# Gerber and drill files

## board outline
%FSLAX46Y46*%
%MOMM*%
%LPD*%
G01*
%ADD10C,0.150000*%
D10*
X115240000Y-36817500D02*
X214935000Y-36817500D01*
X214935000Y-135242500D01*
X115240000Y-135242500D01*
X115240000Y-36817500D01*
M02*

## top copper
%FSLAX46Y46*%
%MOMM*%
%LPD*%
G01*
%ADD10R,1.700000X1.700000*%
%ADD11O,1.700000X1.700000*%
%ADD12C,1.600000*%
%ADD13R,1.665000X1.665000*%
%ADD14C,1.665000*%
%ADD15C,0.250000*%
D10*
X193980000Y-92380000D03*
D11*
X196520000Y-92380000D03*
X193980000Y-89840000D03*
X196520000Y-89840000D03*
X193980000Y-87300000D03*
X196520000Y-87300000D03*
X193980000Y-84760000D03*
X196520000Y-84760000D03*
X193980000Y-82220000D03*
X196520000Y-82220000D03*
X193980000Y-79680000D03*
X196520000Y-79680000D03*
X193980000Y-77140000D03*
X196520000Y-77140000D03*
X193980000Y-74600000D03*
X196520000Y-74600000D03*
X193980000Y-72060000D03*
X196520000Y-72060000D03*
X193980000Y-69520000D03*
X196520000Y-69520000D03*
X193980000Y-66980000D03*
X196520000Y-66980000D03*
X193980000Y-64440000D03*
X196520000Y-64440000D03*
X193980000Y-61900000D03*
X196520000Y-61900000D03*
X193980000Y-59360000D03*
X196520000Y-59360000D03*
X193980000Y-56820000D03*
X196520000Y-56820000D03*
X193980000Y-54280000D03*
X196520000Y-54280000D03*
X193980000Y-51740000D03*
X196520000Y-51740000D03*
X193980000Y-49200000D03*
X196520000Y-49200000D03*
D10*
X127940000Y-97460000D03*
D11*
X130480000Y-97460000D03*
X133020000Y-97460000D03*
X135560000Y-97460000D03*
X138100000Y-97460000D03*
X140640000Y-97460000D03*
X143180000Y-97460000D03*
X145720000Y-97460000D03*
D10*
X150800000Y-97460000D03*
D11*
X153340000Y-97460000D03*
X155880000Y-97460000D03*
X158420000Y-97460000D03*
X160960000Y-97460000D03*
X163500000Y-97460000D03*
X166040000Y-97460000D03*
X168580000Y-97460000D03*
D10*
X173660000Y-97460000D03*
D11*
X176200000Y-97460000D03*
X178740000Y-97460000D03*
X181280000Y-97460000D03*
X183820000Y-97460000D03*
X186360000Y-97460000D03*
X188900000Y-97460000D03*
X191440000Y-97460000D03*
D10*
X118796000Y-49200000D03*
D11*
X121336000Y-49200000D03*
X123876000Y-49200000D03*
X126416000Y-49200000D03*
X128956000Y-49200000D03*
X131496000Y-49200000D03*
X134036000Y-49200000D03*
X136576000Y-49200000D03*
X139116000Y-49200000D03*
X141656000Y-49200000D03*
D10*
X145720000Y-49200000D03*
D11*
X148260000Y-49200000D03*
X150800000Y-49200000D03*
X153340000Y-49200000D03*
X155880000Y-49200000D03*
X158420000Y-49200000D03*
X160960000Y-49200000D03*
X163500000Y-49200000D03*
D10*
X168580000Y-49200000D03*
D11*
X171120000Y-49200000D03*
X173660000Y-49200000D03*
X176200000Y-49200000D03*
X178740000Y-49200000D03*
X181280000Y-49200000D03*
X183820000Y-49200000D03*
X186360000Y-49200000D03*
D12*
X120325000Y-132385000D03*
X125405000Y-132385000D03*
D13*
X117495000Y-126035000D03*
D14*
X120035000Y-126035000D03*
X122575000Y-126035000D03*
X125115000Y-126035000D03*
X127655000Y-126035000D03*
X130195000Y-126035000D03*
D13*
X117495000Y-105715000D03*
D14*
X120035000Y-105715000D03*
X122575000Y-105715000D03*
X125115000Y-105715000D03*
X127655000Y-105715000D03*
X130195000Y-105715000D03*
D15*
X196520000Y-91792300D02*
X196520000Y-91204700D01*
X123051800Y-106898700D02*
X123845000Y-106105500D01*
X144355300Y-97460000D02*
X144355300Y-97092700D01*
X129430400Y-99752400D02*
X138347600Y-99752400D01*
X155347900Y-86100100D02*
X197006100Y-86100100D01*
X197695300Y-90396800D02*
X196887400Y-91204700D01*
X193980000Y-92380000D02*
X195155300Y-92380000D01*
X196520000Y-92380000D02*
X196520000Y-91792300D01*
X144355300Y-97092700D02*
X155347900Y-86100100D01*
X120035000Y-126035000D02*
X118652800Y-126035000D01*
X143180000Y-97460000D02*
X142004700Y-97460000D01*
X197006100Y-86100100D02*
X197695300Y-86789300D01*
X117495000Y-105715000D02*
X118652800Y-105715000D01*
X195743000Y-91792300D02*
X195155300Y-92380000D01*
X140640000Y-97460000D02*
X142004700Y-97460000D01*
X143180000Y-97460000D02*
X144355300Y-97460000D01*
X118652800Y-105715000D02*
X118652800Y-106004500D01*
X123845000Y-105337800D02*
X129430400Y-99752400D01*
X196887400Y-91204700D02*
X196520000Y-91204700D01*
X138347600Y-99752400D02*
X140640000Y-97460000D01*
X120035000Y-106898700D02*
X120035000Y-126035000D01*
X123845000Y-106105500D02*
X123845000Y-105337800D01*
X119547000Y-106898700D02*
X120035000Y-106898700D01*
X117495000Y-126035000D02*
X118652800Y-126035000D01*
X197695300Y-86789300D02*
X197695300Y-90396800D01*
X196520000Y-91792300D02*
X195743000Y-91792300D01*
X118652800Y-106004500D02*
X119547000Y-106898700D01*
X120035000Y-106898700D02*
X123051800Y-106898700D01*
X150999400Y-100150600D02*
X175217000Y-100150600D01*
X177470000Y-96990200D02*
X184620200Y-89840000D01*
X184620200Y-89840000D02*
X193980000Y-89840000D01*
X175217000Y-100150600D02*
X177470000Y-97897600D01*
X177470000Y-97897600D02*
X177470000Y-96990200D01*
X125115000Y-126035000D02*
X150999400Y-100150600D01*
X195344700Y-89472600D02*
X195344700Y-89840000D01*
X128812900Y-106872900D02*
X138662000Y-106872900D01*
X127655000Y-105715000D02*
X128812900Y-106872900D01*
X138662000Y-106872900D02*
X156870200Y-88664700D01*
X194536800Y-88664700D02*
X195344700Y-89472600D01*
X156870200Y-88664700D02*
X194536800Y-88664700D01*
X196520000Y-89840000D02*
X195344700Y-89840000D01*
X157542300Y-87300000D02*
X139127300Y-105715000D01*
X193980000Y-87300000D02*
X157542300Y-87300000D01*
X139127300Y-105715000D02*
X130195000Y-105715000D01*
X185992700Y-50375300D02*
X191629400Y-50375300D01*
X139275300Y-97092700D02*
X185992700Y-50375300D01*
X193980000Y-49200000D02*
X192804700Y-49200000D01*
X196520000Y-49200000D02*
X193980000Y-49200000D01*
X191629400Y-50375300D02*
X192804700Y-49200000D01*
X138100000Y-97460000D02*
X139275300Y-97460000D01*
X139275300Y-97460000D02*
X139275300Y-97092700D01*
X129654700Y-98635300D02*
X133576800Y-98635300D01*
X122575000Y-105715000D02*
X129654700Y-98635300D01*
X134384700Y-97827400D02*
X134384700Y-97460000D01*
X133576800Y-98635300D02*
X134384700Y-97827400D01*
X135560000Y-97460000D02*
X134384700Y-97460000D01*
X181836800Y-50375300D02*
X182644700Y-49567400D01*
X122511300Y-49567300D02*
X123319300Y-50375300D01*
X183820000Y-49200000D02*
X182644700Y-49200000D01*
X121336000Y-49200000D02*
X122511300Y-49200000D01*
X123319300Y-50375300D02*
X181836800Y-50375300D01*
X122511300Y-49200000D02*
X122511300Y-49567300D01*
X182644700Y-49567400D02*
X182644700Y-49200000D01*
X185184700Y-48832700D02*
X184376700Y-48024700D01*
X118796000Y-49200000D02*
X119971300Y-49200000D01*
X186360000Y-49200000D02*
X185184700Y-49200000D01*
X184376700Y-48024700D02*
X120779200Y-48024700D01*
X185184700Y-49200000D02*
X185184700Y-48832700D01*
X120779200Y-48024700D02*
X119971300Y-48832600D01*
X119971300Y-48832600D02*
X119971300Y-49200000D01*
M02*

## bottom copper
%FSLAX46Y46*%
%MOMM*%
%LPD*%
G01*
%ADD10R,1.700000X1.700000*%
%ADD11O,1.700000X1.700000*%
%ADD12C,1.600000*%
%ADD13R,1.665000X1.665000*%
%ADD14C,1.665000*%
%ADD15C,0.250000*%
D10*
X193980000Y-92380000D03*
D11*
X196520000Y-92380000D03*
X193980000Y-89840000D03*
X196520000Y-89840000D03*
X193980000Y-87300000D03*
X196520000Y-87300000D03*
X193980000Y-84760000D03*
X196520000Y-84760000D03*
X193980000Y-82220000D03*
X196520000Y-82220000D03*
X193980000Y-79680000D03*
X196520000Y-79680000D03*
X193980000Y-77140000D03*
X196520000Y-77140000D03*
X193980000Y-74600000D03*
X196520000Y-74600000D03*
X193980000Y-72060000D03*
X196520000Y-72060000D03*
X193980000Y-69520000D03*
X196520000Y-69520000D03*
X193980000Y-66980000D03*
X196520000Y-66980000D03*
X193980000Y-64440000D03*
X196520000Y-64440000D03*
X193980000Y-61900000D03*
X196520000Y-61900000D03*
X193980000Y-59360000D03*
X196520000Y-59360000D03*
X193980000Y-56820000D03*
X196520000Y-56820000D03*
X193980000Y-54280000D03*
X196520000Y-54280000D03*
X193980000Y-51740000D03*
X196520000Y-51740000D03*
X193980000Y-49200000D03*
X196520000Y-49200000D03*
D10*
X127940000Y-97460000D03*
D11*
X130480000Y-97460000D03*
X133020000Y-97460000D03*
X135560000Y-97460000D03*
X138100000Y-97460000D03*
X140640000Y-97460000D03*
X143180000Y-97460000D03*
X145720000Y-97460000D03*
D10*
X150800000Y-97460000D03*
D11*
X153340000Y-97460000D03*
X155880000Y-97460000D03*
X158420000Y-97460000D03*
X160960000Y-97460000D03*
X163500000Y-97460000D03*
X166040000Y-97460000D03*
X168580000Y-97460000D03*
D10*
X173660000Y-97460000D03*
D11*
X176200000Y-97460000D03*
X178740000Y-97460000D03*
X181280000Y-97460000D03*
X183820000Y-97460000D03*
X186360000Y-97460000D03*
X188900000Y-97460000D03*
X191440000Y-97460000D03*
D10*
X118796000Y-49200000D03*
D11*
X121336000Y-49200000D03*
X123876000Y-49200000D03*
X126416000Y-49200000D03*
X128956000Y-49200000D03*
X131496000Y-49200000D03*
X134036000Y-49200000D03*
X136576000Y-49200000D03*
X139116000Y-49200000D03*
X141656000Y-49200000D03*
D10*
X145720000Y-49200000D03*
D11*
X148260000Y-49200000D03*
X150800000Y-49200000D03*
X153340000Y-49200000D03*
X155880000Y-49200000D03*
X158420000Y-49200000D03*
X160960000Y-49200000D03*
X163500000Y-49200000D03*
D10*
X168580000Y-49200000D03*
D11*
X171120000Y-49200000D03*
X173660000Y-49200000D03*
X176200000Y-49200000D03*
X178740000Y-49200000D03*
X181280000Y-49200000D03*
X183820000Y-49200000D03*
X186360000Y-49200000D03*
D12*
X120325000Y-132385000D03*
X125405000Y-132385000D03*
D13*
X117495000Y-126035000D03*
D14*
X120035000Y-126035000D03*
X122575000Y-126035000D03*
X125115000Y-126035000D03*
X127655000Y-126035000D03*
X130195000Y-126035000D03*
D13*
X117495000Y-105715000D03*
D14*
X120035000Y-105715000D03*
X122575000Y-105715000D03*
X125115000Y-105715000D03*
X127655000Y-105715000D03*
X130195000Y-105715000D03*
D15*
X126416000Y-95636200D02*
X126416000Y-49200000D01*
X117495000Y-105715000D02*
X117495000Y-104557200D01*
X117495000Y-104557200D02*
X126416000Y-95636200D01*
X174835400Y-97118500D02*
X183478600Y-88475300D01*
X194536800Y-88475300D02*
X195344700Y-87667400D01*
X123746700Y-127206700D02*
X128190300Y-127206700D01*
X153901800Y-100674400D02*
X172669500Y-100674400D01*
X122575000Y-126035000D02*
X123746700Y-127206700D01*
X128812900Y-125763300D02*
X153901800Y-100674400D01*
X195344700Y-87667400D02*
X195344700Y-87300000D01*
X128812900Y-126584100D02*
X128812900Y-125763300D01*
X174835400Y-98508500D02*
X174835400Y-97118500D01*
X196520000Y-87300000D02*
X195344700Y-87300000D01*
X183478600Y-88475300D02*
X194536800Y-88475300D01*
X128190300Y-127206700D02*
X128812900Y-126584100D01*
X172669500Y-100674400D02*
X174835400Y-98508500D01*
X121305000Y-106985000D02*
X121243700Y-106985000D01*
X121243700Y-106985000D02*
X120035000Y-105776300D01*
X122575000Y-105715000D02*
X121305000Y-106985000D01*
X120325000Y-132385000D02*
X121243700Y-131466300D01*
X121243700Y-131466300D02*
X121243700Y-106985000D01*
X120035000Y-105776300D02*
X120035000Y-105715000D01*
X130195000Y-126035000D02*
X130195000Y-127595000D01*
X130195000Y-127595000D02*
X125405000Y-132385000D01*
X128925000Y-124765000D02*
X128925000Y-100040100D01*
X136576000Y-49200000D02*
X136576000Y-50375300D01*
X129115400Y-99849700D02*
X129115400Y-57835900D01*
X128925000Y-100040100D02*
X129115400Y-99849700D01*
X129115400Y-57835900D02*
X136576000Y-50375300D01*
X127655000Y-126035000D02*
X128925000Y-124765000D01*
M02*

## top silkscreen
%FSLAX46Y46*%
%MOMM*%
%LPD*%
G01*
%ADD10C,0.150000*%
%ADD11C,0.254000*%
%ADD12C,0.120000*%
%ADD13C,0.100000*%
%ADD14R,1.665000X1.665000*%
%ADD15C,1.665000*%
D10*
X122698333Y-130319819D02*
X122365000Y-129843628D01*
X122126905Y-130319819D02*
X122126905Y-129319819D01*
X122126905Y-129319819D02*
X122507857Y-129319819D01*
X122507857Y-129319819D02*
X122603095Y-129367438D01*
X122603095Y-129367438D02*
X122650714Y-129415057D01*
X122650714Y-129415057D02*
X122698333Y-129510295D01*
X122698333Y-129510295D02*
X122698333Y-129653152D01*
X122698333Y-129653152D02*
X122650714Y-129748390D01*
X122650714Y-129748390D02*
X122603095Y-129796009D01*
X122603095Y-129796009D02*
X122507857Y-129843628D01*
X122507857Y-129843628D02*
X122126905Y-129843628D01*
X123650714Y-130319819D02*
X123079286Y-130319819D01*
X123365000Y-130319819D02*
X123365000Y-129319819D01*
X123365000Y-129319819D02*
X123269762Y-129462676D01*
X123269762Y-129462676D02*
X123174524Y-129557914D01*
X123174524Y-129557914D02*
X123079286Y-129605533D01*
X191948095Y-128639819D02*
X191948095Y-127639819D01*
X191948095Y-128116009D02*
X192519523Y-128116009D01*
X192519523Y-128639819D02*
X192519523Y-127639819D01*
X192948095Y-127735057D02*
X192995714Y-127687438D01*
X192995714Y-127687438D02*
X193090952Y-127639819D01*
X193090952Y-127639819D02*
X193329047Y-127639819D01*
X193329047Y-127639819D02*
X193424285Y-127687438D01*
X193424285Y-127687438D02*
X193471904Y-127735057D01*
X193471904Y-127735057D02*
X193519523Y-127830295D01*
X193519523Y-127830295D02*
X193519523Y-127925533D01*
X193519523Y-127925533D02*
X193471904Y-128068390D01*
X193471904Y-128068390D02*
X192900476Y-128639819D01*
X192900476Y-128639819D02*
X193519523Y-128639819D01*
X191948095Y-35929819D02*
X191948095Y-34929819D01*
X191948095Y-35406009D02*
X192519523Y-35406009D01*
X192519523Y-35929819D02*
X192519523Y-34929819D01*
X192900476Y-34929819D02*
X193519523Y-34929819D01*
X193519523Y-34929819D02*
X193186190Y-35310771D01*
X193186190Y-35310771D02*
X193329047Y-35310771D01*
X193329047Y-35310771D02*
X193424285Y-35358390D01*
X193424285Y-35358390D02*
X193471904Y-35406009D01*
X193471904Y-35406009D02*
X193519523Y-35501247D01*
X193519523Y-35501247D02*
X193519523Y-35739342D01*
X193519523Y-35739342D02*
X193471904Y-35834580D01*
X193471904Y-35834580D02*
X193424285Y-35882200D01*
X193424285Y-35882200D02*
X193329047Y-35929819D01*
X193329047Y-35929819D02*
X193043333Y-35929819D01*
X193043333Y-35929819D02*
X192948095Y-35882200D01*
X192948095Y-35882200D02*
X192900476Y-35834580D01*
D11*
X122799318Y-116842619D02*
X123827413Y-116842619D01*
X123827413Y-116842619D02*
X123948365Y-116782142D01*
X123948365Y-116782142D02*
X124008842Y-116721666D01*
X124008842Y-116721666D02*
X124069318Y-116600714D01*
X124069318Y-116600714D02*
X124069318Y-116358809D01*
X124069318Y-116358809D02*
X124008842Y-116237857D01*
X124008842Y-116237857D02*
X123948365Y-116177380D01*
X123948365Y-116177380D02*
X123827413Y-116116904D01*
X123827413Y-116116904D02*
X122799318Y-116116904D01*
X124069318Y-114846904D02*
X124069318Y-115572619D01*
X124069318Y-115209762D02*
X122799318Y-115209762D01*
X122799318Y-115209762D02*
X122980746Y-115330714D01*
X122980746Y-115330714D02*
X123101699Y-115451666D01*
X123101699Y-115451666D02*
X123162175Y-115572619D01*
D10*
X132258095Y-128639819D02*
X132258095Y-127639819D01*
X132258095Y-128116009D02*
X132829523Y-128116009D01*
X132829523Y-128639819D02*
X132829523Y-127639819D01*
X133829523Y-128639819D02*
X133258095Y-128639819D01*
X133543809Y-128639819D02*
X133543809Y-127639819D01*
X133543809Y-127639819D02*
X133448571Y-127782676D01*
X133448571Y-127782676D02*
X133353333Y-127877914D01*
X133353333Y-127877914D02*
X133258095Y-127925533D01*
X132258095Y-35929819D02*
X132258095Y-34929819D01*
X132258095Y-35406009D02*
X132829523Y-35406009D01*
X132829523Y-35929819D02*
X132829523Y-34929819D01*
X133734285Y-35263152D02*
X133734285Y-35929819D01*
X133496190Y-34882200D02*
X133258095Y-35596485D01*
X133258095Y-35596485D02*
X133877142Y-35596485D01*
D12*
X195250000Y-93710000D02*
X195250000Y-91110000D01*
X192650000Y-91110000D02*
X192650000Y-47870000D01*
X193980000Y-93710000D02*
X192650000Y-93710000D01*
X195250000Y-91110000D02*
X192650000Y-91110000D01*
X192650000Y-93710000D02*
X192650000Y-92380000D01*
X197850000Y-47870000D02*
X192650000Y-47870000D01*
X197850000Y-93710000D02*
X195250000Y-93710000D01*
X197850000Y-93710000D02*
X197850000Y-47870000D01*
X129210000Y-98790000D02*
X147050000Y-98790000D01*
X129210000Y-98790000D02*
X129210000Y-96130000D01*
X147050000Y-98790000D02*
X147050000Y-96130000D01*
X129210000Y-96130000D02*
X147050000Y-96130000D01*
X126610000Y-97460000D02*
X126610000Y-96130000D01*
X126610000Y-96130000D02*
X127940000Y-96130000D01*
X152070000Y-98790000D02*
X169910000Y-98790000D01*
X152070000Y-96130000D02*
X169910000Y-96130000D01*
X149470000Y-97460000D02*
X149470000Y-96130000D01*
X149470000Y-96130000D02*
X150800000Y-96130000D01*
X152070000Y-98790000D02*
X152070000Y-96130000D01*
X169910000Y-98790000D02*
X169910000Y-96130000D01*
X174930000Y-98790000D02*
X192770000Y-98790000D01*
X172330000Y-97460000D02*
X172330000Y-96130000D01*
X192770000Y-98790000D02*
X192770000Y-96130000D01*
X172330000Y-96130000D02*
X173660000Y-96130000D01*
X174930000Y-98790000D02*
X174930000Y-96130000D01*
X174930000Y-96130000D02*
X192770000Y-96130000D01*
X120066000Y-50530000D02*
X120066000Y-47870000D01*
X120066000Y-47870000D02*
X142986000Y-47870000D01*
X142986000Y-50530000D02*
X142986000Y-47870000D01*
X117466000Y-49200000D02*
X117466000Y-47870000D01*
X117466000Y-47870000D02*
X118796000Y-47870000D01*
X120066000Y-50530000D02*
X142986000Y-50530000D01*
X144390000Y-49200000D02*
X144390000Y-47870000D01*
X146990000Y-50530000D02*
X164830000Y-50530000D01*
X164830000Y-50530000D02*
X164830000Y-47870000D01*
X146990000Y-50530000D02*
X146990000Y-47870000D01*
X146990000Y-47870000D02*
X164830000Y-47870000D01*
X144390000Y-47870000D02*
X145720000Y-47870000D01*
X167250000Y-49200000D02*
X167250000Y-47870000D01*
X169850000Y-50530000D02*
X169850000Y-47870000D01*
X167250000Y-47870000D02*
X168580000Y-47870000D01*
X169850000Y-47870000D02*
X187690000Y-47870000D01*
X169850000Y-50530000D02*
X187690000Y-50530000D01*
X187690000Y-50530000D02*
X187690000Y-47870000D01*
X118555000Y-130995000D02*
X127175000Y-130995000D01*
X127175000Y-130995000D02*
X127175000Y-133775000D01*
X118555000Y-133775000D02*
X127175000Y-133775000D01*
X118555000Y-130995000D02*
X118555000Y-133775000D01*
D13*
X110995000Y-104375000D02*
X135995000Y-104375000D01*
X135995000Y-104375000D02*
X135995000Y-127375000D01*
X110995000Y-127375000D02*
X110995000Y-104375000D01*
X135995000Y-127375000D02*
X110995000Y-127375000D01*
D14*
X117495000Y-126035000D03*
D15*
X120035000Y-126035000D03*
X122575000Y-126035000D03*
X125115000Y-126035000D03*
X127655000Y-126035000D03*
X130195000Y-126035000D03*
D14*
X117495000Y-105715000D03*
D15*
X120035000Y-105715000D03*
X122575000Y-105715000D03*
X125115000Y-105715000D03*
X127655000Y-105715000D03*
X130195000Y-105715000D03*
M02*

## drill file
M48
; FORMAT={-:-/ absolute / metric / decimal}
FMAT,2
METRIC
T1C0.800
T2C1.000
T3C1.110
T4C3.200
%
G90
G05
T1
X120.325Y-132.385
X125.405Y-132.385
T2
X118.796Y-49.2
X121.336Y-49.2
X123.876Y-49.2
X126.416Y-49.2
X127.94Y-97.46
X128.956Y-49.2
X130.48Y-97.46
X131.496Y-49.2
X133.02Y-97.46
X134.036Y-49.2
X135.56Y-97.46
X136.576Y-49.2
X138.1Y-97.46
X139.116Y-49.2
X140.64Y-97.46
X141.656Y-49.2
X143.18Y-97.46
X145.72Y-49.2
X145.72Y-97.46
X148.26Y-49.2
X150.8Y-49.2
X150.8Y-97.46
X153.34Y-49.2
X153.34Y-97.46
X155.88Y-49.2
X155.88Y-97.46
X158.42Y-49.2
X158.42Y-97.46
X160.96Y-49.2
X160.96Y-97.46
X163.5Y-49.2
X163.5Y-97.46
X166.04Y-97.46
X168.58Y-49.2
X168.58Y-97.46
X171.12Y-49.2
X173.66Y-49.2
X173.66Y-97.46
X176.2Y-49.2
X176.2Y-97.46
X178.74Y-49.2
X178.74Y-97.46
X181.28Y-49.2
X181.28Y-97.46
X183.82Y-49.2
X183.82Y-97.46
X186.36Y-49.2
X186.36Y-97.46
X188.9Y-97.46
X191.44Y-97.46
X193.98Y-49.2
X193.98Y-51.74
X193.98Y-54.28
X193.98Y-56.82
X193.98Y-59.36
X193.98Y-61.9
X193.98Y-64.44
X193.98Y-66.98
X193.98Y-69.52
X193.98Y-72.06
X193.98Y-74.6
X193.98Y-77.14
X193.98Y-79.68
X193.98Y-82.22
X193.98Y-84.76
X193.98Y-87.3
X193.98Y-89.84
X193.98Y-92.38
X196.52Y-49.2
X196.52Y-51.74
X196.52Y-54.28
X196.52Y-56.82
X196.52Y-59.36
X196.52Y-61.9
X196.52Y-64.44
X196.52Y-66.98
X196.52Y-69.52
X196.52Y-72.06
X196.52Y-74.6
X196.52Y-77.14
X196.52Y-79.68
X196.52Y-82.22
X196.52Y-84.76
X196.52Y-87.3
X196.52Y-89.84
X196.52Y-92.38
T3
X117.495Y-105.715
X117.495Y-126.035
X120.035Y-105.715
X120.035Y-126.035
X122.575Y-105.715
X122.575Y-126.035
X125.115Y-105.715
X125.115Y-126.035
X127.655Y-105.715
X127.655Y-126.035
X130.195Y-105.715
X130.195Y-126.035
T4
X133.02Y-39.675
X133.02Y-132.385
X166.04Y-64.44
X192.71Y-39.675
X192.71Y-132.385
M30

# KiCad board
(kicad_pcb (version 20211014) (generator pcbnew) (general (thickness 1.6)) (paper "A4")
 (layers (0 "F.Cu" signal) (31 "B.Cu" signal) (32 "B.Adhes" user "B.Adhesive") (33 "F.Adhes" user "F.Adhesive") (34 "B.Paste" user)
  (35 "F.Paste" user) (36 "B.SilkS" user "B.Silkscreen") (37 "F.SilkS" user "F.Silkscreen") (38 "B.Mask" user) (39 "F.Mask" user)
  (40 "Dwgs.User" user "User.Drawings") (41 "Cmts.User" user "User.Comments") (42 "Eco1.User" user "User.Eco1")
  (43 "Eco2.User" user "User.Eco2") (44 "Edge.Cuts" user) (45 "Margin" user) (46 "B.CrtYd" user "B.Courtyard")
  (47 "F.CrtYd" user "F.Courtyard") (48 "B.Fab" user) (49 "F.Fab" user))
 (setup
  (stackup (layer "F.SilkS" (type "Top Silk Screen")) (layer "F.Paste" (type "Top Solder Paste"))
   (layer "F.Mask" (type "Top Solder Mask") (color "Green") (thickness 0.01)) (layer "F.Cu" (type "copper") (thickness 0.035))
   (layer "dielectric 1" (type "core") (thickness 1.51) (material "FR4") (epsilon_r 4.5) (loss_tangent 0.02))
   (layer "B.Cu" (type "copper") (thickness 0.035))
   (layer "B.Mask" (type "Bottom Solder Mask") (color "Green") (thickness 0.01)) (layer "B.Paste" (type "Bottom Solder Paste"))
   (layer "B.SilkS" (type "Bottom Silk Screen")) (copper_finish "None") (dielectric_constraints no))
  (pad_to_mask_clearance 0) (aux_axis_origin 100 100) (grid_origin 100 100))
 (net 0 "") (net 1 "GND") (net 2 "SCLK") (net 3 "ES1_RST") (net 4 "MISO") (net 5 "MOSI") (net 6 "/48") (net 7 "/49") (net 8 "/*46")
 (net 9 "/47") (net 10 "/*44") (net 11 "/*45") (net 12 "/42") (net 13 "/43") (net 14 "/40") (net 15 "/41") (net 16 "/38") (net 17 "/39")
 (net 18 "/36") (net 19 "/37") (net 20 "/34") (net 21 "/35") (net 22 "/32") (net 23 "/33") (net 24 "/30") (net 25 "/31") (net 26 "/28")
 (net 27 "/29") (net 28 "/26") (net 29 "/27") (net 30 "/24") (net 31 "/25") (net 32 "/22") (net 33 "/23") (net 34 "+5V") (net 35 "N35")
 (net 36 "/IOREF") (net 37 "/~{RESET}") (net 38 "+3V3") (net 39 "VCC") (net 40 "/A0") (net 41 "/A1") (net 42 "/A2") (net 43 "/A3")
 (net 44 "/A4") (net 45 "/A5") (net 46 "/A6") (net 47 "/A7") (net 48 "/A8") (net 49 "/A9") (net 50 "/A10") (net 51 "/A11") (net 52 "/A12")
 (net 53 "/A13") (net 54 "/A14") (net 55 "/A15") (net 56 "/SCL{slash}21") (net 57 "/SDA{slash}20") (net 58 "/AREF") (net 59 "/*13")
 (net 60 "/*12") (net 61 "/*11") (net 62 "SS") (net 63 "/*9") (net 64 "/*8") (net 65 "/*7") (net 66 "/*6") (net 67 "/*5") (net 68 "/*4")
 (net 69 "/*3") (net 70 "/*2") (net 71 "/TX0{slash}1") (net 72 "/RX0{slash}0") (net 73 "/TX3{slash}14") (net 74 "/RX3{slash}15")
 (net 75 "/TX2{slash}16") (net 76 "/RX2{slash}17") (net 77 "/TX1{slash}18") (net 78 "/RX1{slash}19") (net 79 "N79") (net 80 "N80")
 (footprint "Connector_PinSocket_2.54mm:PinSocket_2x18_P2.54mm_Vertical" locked (layer "F.Cu") (at 193.98 92.38 180)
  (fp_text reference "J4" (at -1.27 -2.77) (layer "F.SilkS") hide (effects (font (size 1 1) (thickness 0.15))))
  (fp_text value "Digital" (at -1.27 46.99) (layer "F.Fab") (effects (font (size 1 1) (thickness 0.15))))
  (fp_line (start -1.27 -1.33) (end -1.27 1.27) (layer "F.SilkS") (width 0.12))
  (fp_line (start 1.33 1.27) (end 1.33 44.51) (layer "F.SilkS") (width 0.12))
  (fp_line (start 0 -1.33) (end 1.33 -1.33) (layer "F.SilkS") (width 0.12))
  (fp_line (start -1.27 1.27) (end 1.33 1.27) (layer "F.SilkS") (width 0.12))
  (fp_line (start 1.33 -1.33) (end 1.33 0) (layer "F.SilkS") (width 0.12))
  (fp_line (start -3.87 44.51) (end 1.33 44.51) (layer "F.SilkS") (width 0.12))
  (fp_line (start -3.87 -1.33) (end -1.27 -1.33) (layer "F.SilkS") (width 0.12))
  (fp_line (start -3.87 -1.33) (end -3.87 44.51) (layer "F.SilkS") (width 0.12))
  (pad "1" thru_hole rect locked (at 0 0 180) (size 1.7 1.7) (drill 1) (layers *.Cu *.Mask) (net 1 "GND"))
  (pad "2" thru_hole oval locked (at -2.54 0 180) (size 1.7 1.7) (drill 1) (layers *.Cu *.Mask) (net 1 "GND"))
  (pad "3" thru_hole oval locked (at 0 2.54 180) (size 1.7 1.7) (drill 1) (layers *.Cu *.Mask) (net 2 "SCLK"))
  (pad "4" thru_hole oval locked (at -2.54 2.54 180) (size 1.7 1.7) (drill 1) (layers *.Cu *.Mask) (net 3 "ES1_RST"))
  (pad "5" thru_hole oval locked (at 0 5.08 180) (size 1.7 1.7) (drill 1) (layers *.Cu *.Mask) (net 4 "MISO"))
  (pad "6" thru_hole oval locked (at -2.54 5.08 180) (size 1.7 1.7) (drill 1) (layers *.Cu *.Mask) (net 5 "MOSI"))
  (pad "7" thru_hole oval locked (at 0 7.62 180) (size 1.7 1.7) (drill 1) (layers *.Cu *.Mask) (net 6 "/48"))
  (pad "8" thru_hole oval locked (at -2.54 7.62 180) (size 1.7 1.7) (drill 1) (layers *.Cu *.Mask) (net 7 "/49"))
  (pad "9" thru_hole oval locked (at 0 10.16 180) (size 1.7 1.7) (drill 1) (layers *.Cu *.Mask) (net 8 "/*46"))
  (pad "10" thru_hole oval locked (at -2.54 10.16 180) (size 1.7 1.7) (drill 1) (layers *.Cu *.Mask) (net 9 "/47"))
  (pad "11" thru_hole oval locked (at 0 12.7 180) (size 1.7 1.7) (drill 1) (layers *.Cu *.Mask) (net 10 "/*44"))
  (pad "12" thru_hole oval locked (at -2.54 12.7 180) (size 1.7 1.7) (drill 1) (layers *.Cu *.Mask) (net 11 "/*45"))
  (pad "13" thru_hole oval locked (at 0 15.24 180) (size 1.7 1.7) (drill 1) (layers *.Cu *.Mask) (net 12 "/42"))
  (pad "14" thru_hole oval locked (at -2.54 15.24 180) (size 1.7 1.7) (drill 1) (layers *.Cu *.Mask) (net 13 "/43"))
  (pad "15" thru_hole oval locked (at 0 17.78 180) (size 1.7 1.7) (drill 1) (layers *.Cu *.Mask) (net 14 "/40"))
  (pad "16" thru_hole oval locked (at -2.54 17.78 180) (size 1.7 1.7) (drill 1) (layers *.Cu *.Mask) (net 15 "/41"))
  (pad "17" thru_hole oval locked (at 0 20.32 180) (size 1.7 1.7) (drill 1) (layers *.Cu *.Mask) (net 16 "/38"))
  (pad "18" thru_hole oval locked (at -2.54 20.32 180) (size 1.7 1.7) (drill 1) (layers *.Cu *.Mask) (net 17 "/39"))
  (pad "19" thru_hole oval locked (at 0 22.86 180) (size 1.7 1.7) (drill 1) (layers *.Cu *.Mask) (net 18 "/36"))
  (pad "20" thru_hole oval locked (at -2.54 22.86 180) (size 1.7 1.7) (drill 1) (layers *.Cu *.Mask) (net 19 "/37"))
  (pad "21" thru_hole oval locked (at 0 25.4 180) (size 1.7 1.7) (drill 1) (layers *.Cu *.Mask) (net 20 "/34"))
  (pad "22" thru_hole oval locked (at -2.54 25.4 180) (size 1.7 1.7) (drill 1) (layers *.Cu *.Mask) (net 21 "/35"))
  (pad "23" thru_hole oval locked (at 0 27.94 180) (size 1.7 1.7) (drill 1) (layers *.Cu *.Mask) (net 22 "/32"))
  (pad "24" thru_hole oval locked (at -2.54 27.94 180) (size 1.7 1.7) (drill 1) (layers *.Cu *.Mask) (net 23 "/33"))
  (pad "25" thru_hole oval locked (at 0 30.48 180) (size 1.7 1.7) (drill 1) (layers *.Cu *.Mask) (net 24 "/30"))
  (pad "26" thru_hole oval locked (at -2.54 30.48 180) (size 1.7 1.7) (drill 1) (layers *.Cu *.Mask) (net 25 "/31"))
  (pad "27" thru_hole oval locked (at 0 33.02 180) (size 1.7 1.7) (drill 1) (layers *.Cu *.Mask) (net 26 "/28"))
  (pad "28" thru_hole oval locked (at -2.54 33.02 180) (size 1.7 1.7) (drill 1) (layers *.Cu *.Mask) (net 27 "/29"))
  (pad "29" thru_hole oval locked (at 0 35.56 180) (size 1.7 1.7) (drill 1) (layers *.Cu *.Mask) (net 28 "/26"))
  (pad "30" thru_hole oval locked (at -2.54 35.56 180) (size 1.7 1.7) (drill 1) (layers *.Cu *.Mask) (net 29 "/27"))
  (pad "31" thru_hole oval locked (at 0 38.1 180) (size 1.7 1.7) (drill 1) (layers *.Cu *.Mask) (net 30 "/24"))
  (pad "32" thru_hole oval locked (at -2.54 38.1 180) (size 1.7 1.7) (drill 1) (layers *.Cu *.Mask) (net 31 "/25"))
  (pad "33" thru_hole oval locked (at 0 40.64 180) (size 1.7 1.7) (drill 1) (layers *.Cu *.Mask) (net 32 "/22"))
  (pad "34" thru_hole oval locked (at -2.54 40.64 180) (size 1.7 1.7) (drill 1) (layers *.Cu *.Mask) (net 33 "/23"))
  (pad "35" thru_hole oval locked (at 0 43.18 180) (size 1.7 1.7) (drill 1) (layers *.Cu *.Mask) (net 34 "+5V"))
  (pad "36" thru_hole oval locked (at -2.54 43.18 180) (size 1.7 1.7) (drill 1) (layers *.Cu *.Mask) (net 34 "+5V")))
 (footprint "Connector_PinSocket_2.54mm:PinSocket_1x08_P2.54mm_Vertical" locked (layer "F.Cu") (at 127.94 97.46 90)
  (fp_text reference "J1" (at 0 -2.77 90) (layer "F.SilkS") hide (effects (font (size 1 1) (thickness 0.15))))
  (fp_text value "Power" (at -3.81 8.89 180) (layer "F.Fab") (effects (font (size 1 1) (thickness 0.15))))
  (fp_line (start -1.33 1.27) (end -1.33 19.11) (layer "F.SilkS") (width 0.12))
  (fp_line (start -1.33 1.27) (end 1.33 1.27) (layer "F.SilkS") (width 0.12))
  (fp_line (start -1.33 19.11) (end 1.33 19.11) (layer "F.SilkS") (width 0.12))
  (fp_line (start 1.33 1.27) (end 1.33 19.11) (layer "F.SilkS") (width 0.12))
  (fp_line (start 0 -1.33) (end 1.33 -1.33) (layer "F.SilkS") (width 0.12))
  (fp_line (start 1.33 -1.33) (end 1.33 0) (layer "F.SilkS") (width 0.12))
  (pad "1" thru_hole rect locked (at 0 0 90) (size 1.7 1.7) (drill 1) (layers *.Cu *.Mask) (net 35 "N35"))
  (pad "2" thru_hole oval locked (at 0 2.54 90) (size 1.7 1.7) (drill 1) (layers *.Cu *.Mask) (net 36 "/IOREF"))
  (pad "3" thru_hole oval locked (at 0 5.08 90) (size 1.7 1.7) (drill 1) (layers *.Cu *.Mask) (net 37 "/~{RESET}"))
  (pad "4" thru_hole oval locked (at 0 7.62 90) (size 1.7 1.7) (drill 1) (layers *.Cu *.Mask) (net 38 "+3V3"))
  (pad "5" thru_hole oval locked (at 0 10.16 90) (size 1.7 1.7) (drill 1) (layers *.Cu *.Mask) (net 34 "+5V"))
  (pad "6" thru_hole oval locked (at 0 12.7 90) (size 1.7 1.7) (drill 1) (layers *.Cu *.Mask) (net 1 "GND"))
  (pad "7" thru_hole oval locked (at 0 15.24 90) (size 1.7 1.7) (drill 1) (layers *.Cu *.Mask) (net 1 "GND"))
  (pad "8" thru_hole oval locked (at 0 17.78 90) (size 1.7 1.7) (drill 1) (layers *.Cu *.Mask) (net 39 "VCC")))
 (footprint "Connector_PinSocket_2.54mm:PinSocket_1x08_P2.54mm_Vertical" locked (layer "F.Cu") (at 150.8 97.46 90)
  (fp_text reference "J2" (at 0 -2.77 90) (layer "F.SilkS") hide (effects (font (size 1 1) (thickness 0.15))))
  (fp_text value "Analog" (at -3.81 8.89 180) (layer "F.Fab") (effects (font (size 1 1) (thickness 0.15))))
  (fp_line (start -1.33 1.27) (end -1.33 19.11) (layer "F.SilkS") (width 0.12))
  (fp_line (start 1.33 1.27) (end 1.33 19.11) (layer "F.SilkS") (width 0.12))
  (fp_line (start 0 -1.33) (end 1.33 -1.33) (layer "F.SilkS") (width 0.12))
  (fp_line (start 1.33 -1.33) (end 1.33 0) (layer "F.SilkS") (width 0.12))
  (fp_line (start -1.33 1.27) (end 1.33 1.27) (layer "F.SilkS") (width 0.12))
  (fp_line (start -1.33 19.11) (end 1.33 19.11) (layer "F.SilkS") (width 0.12))
  (pad "1" thru_hole rect locked (at 0 0 90) (size 1.7 1.7) (drill 1) (layers *.Cu *.Mask) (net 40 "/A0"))
  (pad "2" thru_hole oval locked (at 0 2.54 90) (size 1.7 1.7) (drill 1) (layers *.Cu *.Mask) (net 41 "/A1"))
  (pad "3" thru_hole oval locked (at 0 5.08 90) (size 1.7 1.7) (drill 1) (layers *.Cu *.Mask) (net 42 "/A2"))
  (pad "4" thru_hole oval locked (at 0 7.62 90) (size 1.7 1.7) (drill 1) (layers *.Cu *.Mask) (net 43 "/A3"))
  (pad "5" thru_hole oval locked (at 0 10.16 90) (size 1.7 1.7) (drill 1) (layers *.Cu *.Mask) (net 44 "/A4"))
  (pad "6" thru_hole oval locked (at 0 12.7 90) (size 1.7 1.7) (drill 1) (layers *.Cu *.Mask) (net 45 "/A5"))
  (pad "7" thru_hole oval locked (at 0 15.24 90) (size 1.7 1.7) (drill 1) (layers *.Cu *.Mask) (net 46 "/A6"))
  (pad "8" thru_hole oval locked (at 0 17.78 90) (size 1.7 1.7) (drill 1) (layers *.Cu *.Mask) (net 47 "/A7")))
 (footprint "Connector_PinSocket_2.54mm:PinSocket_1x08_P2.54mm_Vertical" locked (layer "F.Cu") (at 173.66 97.46 90)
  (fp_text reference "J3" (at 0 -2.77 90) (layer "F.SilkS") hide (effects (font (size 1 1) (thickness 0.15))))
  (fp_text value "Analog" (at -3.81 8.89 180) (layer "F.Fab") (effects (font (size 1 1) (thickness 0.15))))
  (fp_line (start -1.33 1.27) (end -1.33 19.11) (layer "F.SilkS") (width 0.12))
  (fp_line (start 0 -1.33) (end 1.33 -1.33) (layer "F.SilkS") (width 0.12))
  (fp_line (start -1.33 19.11) (end 1.33 19.11) (layer "F.SilkS") (width 0.12))
  (fp_line (start 1.33 -1.33) (end 1.33 0) (layer "F.SilkS") (width 0.12))
  (fp_line (start -1.33 1.27) (end 1.33 1.27) (layer "F.SilkS") (width 0.12))
  (fp_line (start 1.33 1.27) (end 1.33 19.11) (layer "F.SilkS") (width 0.12))
  (pad "1" thru_hole rect locked (at 0 0 90) (size 1.7 1.7) (drill 1) (layers *.Cu *.Mask) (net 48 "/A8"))
  (pad "2" thru_hole oval locked (at 0 2.54 90) (size 1.7 1.7) (drill 1) (layers *.Cu *.Mask) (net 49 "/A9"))
  (pad "3" thru_hole oval locked (at 0 5.08 90) (size 1.7 1.7) (drill 1) (layers *.Cu *.Mask) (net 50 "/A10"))
  (pad "4" thru_hole oval locked (at 0 7.62 90) (size 1.7 1.7) (drill 1) (layers *.Cu *.Mask) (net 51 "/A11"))
  (pad "5" thru_hole oval locked (at 0 10.16 90) (size 1.7 1.7) (drill 1) (layers *.Cu *.Mask) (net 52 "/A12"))
  (pad "6" thru_hole oval locked (at 0 12.7 90) (size 1.7 1.7) (drill 1) (layers *.Cu *.Mask) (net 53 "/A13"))
  (pad "7" thru_hole oval locked (at 0 15.24 90) (size 1.7 1.7) (drill 1) (layers *.Cu *.Mask) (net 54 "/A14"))
  (pad "8" thru_hole oval locked (at 0 17.78 90) (size 1.7 1.7) (drill 1) (layers *.Cu *.Mask) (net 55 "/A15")))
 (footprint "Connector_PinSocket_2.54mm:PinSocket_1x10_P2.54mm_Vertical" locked (layer "F.Cu") (at 118.796 49.2 90)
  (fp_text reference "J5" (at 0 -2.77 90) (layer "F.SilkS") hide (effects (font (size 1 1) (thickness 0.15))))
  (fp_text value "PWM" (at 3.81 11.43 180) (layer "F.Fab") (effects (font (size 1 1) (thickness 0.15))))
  (fp_line (start -1.33 1.27) (end 1.33 1.27) (layer "F.SilkS") (width 0.12))
  (fp_line (start 1.33 1.27) (end 1.33 24.19) (layer "F.SilkS") (width 0.12))
  (fp_line (start -1.33 24.19) (end 1.33 24.19) (layer "F.SilkS") (width 0.12))
  (fp_line (start 0 -1.33) (end 1.33 -1.33) (layer "F.SilkS") (width 0.12))
  (fp_line (start 1.33 -1.33) (end 1.33 0) (layer "F.SilkS") (width 0.12))
  (fp_line (start -1.33 1.27) (end -1.33 24.19) (layer "F.SilkS") (width 0.12))
  (pad "1" thru_hole rect locked (at 0 0 90) (size 1.7 1.7) (drill 1) (layers *.Cu *.Mask) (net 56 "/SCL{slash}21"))
  (pad "2" thru_hole oval locked (at 0 2.54 90) (size 1.7 1.7) (drill 1) (layers *.Cu *.Mask) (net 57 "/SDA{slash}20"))
  (pad "3" thru_hole oval locked (at 0 5.08 90) (size 1.7 1.7) (drill 1) (layers *.Cu *.Mask) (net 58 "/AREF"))
  (pad "4" thru_hole oval locked (at 0 7.62 90) (size 1.7 1.7) (drill 1) (layers *.Cu *.Mask) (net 1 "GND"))
  (pad "5" thru_hole oval locked (at 0 10.16 90) (size 1.7 1.7) (drill 1) (layers *.Cu *.Mask) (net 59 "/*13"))
  (pad "6" thru_hole oval locked (at 0 12.7 90) (size 1.7 1.7) (drill 1) (layers *.Cu *.Mask) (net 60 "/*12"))
  (pad "7" thru_hole oval locked (at 0 15.24 90) (size 1.7 1.7) (drill 1) (layers *.Cu *.Mask) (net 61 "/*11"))
  (pad "8" thru_hole oval locked (at 0 17.78 90) (size 1.7 1.7) (drill 1) (layers *.Cu *.Mask) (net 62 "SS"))
  (pad "9" thru_hole oval locked (at 0 20.32 90) (size 1.7 1.7) (drill 1) (layers *.Cu *.Mask) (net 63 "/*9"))
  (pad "10" thru_hole oval locked (at 0 22.86 90) (size 1.7 1.7) (drill 1) (layers *.Cu *.Mask) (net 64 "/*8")))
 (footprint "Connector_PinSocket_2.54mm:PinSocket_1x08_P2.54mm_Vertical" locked (layer "F.Cu") (at 145.72 49.2 90)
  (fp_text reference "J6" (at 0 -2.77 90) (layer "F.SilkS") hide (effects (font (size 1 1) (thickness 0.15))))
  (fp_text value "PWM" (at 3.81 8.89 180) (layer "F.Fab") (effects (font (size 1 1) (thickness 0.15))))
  (fp_line (start 0 -1.33) (end 1.33 -1.33) (layer "F.SilkS") (width 0.12))
  (fp_line (start -1.33 1.27) (end -1.33 19.11) (layer "F.SilkS") (width 0.12))
  (fp_line (start -1.33 19.11) (end 1.33 19.11) (layer "F.SilkS") (width 0.12))
  (fp_line (start -1.33 1.27) (end 1.33 1.27) (layer "F.SilkS") (width 0.12))
  (fp_line (start 1.33 1.27) (end 1.33 19.11) (layer "F.SilkS") (width 0.12))
  (fp_line (start 1.33 -1.33) (end 1.33 0) (layer "F.SilkS") (width 0.12))
  (pad "1" thru_hole rect locked (at 0 0 90) (size 1.7 1.7) (drill 1) (layers *.Cu *.Mask) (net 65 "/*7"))
  (pad "2" thru_hole oval locked (at 0 2.54 90) (size 1.7 1.7) (drill 1) (layers *.Cu *.Mask) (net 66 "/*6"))
  (pad "3" thru_hole oval locked (at 0 5.08 90) (size 1.7 1.7) (drill 1) (layers *.Cu *.Mask) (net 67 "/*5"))
  (pad "4" thru_hole oval locked (at 0 7.62 90) (size 1.7 1.7) (drill 1) (layers *.Cu *.Mask) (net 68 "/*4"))
  (pad "5" thru_hole oval locked (at 0 10.16 90) (size 1.7 1.7) (drill 1) (layers *.Cu *.Mask) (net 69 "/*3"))
  (pad "6" thru_hole oval locked (at 0 12.7 90) (size 1.7 1.7) (drill 1) (layers *.Cu *.Mask) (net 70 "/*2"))
  (pad "7" thru_hole oval locked (at 0 15.24 90) (size 1.7 1.7) (drill 1) (layers *.Cu *.Mask) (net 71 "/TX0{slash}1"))
  (pad "8" thru_hole oval locked (at 0 17.78 90) (size 1.7 1.7) (drill 1) (layers *.Cu *.Mask) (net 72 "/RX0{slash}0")))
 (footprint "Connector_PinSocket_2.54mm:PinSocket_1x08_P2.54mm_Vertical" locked (layer "F.Cu") (at 168.58 49.2 90)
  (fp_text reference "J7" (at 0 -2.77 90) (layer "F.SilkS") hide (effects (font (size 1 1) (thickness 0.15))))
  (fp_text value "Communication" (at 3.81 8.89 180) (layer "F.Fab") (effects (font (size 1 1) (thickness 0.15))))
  (fp_line (start 0 -1.33) (end 1.33 -1.33) (layer "F.SilkS") (width 0.12))
  (fp_line (start -1.33 1.27) (end 1.33 1.27) (layer "F.SilkS") (width 0.12))
  (fp_line (start 1.33 -1.33) (end 1.33 0) (layer "F.SilkS") (width 0.12))
  (fp_line (start 1.33 1.27) (end 1.33 19.11) (layer "F.SilkS") (width 0.12))
  (fp_line (start -1.33 1.27) (end -1.33 19.11) (layer "F.SilkS") (width 0.12))
  (fp_line (start -1.33 19.11) (end 1.33 19.11) (layer "F.SilkS") (width 0.12))
  (pad "1" thru_hole rect locked (at 0 0 90) (size 1.7 1.7) (drill 1) (layers *.Cu *.Mask) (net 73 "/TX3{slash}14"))
  (pad "2" thru_hole oval locked (at 0 2.54 90) (size 1.7 1.7) (drill 1) (layers *.Cu *.Mask) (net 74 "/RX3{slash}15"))
  (pad "3" thru_hole oval locked (at 0 5.08 90) (size 1.7 1.7) (drill 1) (layers *.Cu *.Mask) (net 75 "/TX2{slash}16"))
  (pad "4" thru_hole oval locked (at 0 7.62 90) (size 1.7 1.7) (drill 1) (layers *.Cu *.Mask) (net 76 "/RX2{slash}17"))
  (pad "5" thru_hole oval locked (at 0 10.16 90) (size 1.7 1.7) (drill 1) (layers *.Cu *.Mask) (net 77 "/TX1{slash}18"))
  (pad "6" thru_hole oval locked (at 0 12.7 90) (size 1.7 1.7) (drill 1) (layers *.Cu *.Mask) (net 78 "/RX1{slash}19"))
  (pad "7" thru_hole oval locked (at 0 15.24 90) (size 1.7 1.7) (drill 1) (layers *.Cu *.Mask) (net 57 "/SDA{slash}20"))
  (pad "8" thru_hole oval locked (at 0 17.78 90) (size 1.7 1.7) (drill 1) (layers *.Cu *.Mask) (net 56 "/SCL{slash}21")))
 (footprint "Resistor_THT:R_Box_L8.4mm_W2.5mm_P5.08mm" (layer "F.Cu") (at 120.325 132.385)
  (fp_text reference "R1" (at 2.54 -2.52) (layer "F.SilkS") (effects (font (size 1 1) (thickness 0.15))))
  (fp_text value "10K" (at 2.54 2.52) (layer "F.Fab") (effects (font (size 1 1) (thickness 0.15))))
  (fp_line (start -1.77 -1.39) (end 6.85 -1.39) (layer "F.SilkS") (width 0.12))
  (fp_line (start 6.85 -1.39) (end 6.85 1.39) (layer "F.SilkS") (width 0.12))
  (fp_line (start -1.77 1.39) (end 6.85 1.39) (layer "F.SilkS") (width 0.12))
  (fp_line (start -1.77 -1.39) (end -1.77 1.39) (layer "F.SilkS") (width 0.12))
  (pad "1" thru_hole circle (at 0 0) (size 1.6 1.6) (drill 0.8) (layers *.Cu *.Mask) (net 38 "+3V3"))
  (pad "2" thru_hole circle (at 5.08 0) (size 1.6 1.6) (drill 0.8) (layers *.Cu *.Mask) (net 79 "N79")))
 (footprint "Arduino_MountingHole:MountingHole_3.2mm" (layer "F.Cu") (at 192.71 132.385)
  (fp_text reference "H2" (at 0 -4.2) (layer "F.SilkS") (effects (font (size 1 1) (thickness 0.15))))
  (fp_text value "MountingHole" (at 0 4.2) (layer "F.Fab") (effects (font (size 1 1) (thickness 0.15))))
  (pad "" np_thru_hole circle locked (at 0 0) (size 3.2 3.2) (drill 3.2) (layers *.Cu *.Mask)))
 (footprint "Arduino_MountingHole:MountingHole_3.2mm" (layer "F.Cu") (at 192.71 39.675)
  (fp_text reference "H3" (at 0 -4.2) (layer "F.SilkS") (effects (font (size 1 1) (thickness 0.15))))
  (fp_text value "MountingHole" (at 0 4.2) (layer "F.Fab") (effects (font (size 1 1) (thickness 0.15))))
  (pad "" np_thru_hole circle locked (at 0 0) (size 3.2 3.2) (drill 3.2) (layers *.Cu *.Mask)))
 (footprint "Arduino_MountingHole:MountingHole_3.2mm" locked (layer "F.Cu") (at 166.04 64.44)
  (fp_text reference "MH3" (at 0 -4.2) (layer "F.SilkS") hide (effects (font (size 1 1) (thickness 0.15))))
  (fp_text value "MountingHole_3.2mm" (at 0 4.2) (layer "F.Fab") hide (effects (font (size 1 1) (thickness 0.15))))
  (pad "" np_thru_hole circle locked (at 0 0) (size 3.2 3.2) (drill 3.2) (layers *.Cu *.Mask)))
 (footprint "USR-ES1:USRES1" (layer "F.Cu") (at 117.495 126.035 90)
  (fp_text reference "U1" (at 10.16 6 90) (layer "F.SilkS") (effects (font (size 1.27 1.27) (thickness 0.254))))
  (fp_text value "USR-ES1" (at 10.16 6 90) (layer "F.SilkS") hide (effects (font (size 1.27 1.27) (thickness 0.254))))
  (fp_line (start 21.66 -6.5) (end 21.66 18.5) (layer "F.SilkS") (width 0.1))
  (fp_line (start 21.66 18.5) (end -1.34 18.5) (layer "F.SilkS") (width 0.1))
  (fp_line (start -1.34 -6.5) (end 21.66 -6.5) (layer "F.SilkS") (width 0.1))
  (fp_line (start -1.34 18.5) (end -1.34 -6.5) (layer "F.SilkS") (width 0.1))
  (pad "A1" thru_hole rect (at 0 0 180) (size 1.665 1.665) (drill 1.11) (layers *.Cu *.Mask "F.SilkS") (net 1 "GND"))
  (pad "A2" thru_hole circle (at 0 2.54 180) (size 1.665 1.665) (drill 1.11) (layers *.Cu *.Mask "F.SilkS") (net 1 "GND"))
  (pad "A3" thru_hole circle (at 0 5.08 180) (size 1.665 1.665) (drill 1.11) (layers *.Cu *.Mask "F.SilkS") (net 5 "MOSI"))
  (pad "A4" thru_hole circle (at 0 7.62 180) (size 1.665 1.665) (drill 1.11) (layers *.Cu *.Mask "F.SilkS") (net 2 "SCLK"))
  (pad "A5" thru_hole circle (at 0 10.16 180) (size 1.665 1.665) (drill 1.11) (layers *.Cu *.Mask "F.SilkS") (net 62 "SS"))
  (pad "A6" thru_hole circle (at 0 12.7 180) (size 1.665 1.665) (drill 1.11) (layers *.Cu *.Mask "F.SilkS") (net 79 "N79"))
  (pad "B1" thru_hole rect (at 20.32 0 180) (size 1.665 1.665) (drill 1.11) (layers *.Cu *.Mask "F.SilkS") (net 1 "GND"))
  (pad "B2" thru_hole circle (at 20.32 2.54 180) (size 1.665 1.665) (drill 1.11) (layers *.Cu *.Mask "F.SilkS") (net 38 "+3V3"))
  (pad "B3" thru_hole circle (at 20.32 5.08 180) (size 1.665 1.665) (drill 1.11) (layers *.Cu *.Mask "F.SilkS") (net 38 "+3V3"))
  (pad "B4" thru_hole circle (at 20.32 7.62 180) (size 1.665 1.665) (drill 1.11) (layers *.Cu *.Mask "F.SilkS") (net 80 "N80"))
  (pad "B5" thru_hole circle (at 20.32 10.16 180) (size 1.665 1.665) (drill 1.11) (layers *.Cu *.Mask "F.SilkS") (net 3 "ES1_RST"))
  (pad "B6" thru_hole circle (at 20.32 12.7 180) (size 1.665 1.665) (drill 1.11) (layers *.Cu *.Mask "F.SilkS") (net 4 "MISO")))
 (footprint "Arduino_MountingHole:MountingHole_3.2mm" (layer "F.Cu") (at 133.02 132.385)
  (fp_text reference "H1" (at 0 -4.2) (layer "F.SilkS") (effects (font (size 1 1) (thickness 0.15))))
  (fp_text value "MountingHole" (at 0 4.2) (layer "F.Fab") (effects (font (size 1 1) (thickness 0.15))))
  (pad "" np_thru_hole circle locked (at 0 0) (size 3.2 3.2) (drill 3.2) (layers *.Cu *.Mask)))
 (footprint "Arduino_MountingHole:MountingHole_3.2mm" (layer "F.Cu") (at 133.02 39.675)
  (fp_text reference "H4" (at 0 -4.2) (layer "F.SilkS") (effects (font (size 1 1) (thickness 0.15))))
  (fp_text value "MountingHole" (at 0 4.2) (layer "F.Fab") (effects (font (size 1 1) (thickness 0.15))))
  (pad "" np_thru_hole circle locked (at 0 0) (size 3.2 3.2) (drill 3.2) (layers *.Cu *.Mask)))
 (gr_rect (start 115.24 36.8175) (end 214.935 135.2425) (layer "Edge.Cuts") (width 0.15) (fill none))
 (segment (start 196.52 91.7923) (end 196.52 91.2047) (width 0.25) (layer "F.Cu") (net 1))
 (segment (start 123.0518 106.8987) (end 123.845 106.1055) (width 0.25) (layer "F.Cu") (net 1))
 (segment (start 144.3553 97.46) (end 144.3553 97.0927) (width 0.25) (layer "F.Cu") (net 1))
 (segment (start 129.4304 99.7524) (end 138.3476 99.7524) (width 0.25) (layer "F.Cu") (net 1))
 (segment (start 155.3479 86.1001) (end 197.0061 86.1001) (width 0.25) (layer "F.Cu") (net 1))
 (segment (start 197.6953 90.3968) (end 196.8874 91.2047) (width 0.25) (layer "F.Cu") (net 1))
 (segment (start 193.98 92.38) (end 195.1553 92.38) (width 0.25) (layer "F.Cu") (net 1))
 (segment (start 196.52 92.38) (end 196.52 91.7923) (width 0.25) (layer "F.Cu") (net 1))
 (segment (start 144.3553 97.0927) (end 155.3479 86.1001) (width 0.25) (layer "F.Cu") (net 1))
 (segment (start 120.035 126.035) (end 118.6528 126.035) (width 0.25) (layer "F.Cu") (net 1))
 (segment (start 143.18 97.46) (end 142.0047 97.46) (width 0.25) (layer "F.Cu") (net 1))
 (segment (start 197.0061 86.1001) (end 197.6953 86.7893) (width 0.25) (layer "F.Cu") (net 1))
 (segment (start 117.495 105.715) (end 118.6528 105.715) (width 0.25) (layer "F.Cu") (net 1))
 (segment (start 195.743 91.7923) (end 195.1553 92.38) (width 0.25) (layer "F.Cu") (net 1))
 (segment (start 140.64 97.46) (end 142.0047 97.46) (width 0.25) (layer "F.Cu") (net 1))
 (segment (start 143.18 97.46) (end 144.3553 97.46) (width 0.25) (layer "F.Cu") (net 1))
 (segment (start 118.6528 105.715) (end 118.6528 106.0045) (width 0.25) (layer "F.Cu") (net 1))
 (segment (start 123.845 105.3378) (end 129.4304 99.7524) (width 0.25) (layer "F.Cu") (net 1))
 (segment (start 196.8874 91.2047) (end 196.52 91.2047) (width 0.25) (layer "F.Cu") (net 1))
 (segment (start 138.3476 99.7524) (end 140.64 97.46) (width 0.25) (layer "F.Cu") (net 1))
 (segment (start 120.035 106.8987) (end 120.035 126.035) (width 0.25) (layer "F.Cu") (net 1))
 (segment (start 123.845 106.1055) (end 123.845 105.3378) (width 0.25) (layer "F.Cu") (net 1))
 (segment (start 119.547 106.8987) (end 120.035 106.8987) (width 0.25) (layer "F.Cu") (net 1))
 (segment (start 117.495 126.035) (end 118.6528 126.035) (width 0.25) (layer "F.Cu") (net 1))
 (segment (start 197.6953 86.7893) (end 197.6953 90.3968) (width 0.25) (layer "F.Cu") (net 1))
 (segment (start 196.52 91.7923) (end 195.743 91.7923) (width 0.25) (layer "F.Cu") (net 1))
 (segment (start 118.6528 106.0045) (end 119.547 106.8987) (width 0.25) (layer "F.Cu") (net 1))
 (segment (start 120.035 106.8987) (end 123.0518 106.8987) (width 0.25) (layer "F.Cu") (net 1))
 (segment (start 126.416 95.6362) (end 126.416 49.2) (width 0.25) (layer "B.Cu") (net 1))
 (segment (start 117.495 105.715) (end 117.495 104.5572) (width 0.25) (layer "B.Cu") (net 1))
 (segment (start 117.495 104.5572) (end 126.416 95.6362) (width 0.25) (layer "B.Cu") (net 1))
 (segment (start 150.9994 100.1506) (end 175.217 100.1506) (width 0.25) (layer "F.Cu") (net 2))
 (segment (start 177.47 96.9902) (end 184.6202 89.84) (width 0.25) (layer "F.Cu") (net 2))
 (segment (start 184.6202 89.84) (end 193.98 89.84) (width 0.25) (layer "F.Cu") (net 2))
 (segment (start 175.217 100.1506) (end 177.47 97.8976) (width 0.25) (layer "F.Cu") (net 2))
 (segment (start 177.47 97.8976) (end 177.47 96.9902) (width 0.25) (layer "F.Cu") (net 2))
 (segment (start 125.115 126.035) (end 150.9994 100.1506) (width 0.25) (layer "F.Cu") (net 2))
 (segment (start 195.3447 89.4726) (end 195.3447 89.84) (width 0.25) (layer "F.Cu") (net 3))
 (segment (start 128.8129 106.8729) (end 138.662 106.8729) (width 0.25) (layer "F.Cu") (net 3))
 (segment (start 127.655 105.715) (end 128.8129 106.8729) (width 0.25) (layer "F.Cu") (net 3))
 (segment (start 138.662 106.8729) (end 156.8702 88.6647) (width 0.25) (layer "F.Cu") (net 3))
 (segment (start 194.5368 88.6647) (end 195.3447 89.4726) (width 0.25) (layer "F.Cu") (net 3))
 (segment (start 156.8702 88.6647) (end 194.5368 88.6647) (width 0.25) (layer "F.Cu") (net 3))
 (segment (start 196.52 89.84) (end 195.3447 89.84) (width 0.25) (layer "F.Cu") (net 3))
 (segment (start 157.5423 87.3) (end 139.1273 105.715) (width 0.25) (layer "F.Cu") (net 4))
 (segment (start 193.98 87.3) (end 157.5423 87.3) (width 0.25) (layer "F.Cu") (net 4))
 (segment (start 139.1273 105.715) (end 130.195 105.715) (width 0.25) (layer "F.Cu") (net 4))
 (segment (start 174.8354 97.1185) (end 183.4786 88.4753) (width 0.25) (layer "B.Cu") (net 5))
 (segment (start 194.5368 88.4753) (end 195.3447 87.6674) (width 0.25) (layer "B.Cu") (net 5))
 (segment (start 123.7467 127.2067) (end 128.1903 127.2067) (width 0.25) (layer "B.Cu") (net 5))
 (segment (start 153.9018 100.6744) (end 172.6695 100.6744) (width 0.25) (layer "B.Cu") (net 5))
 (segment (start 122.575 126.035) (end 123.7467 127.2067) (width 0.25) (layer "B.Cu") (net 5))
 (segment (start 128.8129 125.7633) (end 153.9018 100.6744) (width 0.25) (layer "B.Cu") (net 5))
 (segment (start 195.3447 87.6674) (end 195.3447 87.3) (width 0.25) (layer "B.Cu") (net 5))
 (segment (start 128.8129 126.5841) (end 128.8129 125.7633) (width 0.25) (layer "B.Cu") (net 5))
 (segment (start 174.8354 98.5085) (end 174.8354 97.1185) (width 0.25) (layer "B.Cu") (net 5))
 (segment (start 196.52 87.3) (end 195.3447 87.3) (width 0.25) (layer "B.Cu") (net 5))
 (segment (start 183.4786 88.4753) (end 194.5368 88.4753) (width 0.25) (layer "B.Cu") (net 5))
 (segment (start 128.1903 127.2067) (end 128.8129 126.5841) (width 0.25) (layer "B.Cu") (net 5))
 (segment (start 172.6695 100.6744) (end 174.8354 98.5085) (width 0.25) (layer "B.Cu") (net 5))
 (segment (start 185.9927 50.3753) (end 191.6294 50.3753) (width 0.25) (layer "F.Cu") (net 34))
 (segment (start 139.2753 97.0927) (end 185.9927 50.3753) (width 0.25) (layer "F.Cu") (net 34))
 (segment (start 193.98 49.2) (end 192.8047 49.2) (width 0.25) (layer "F.Cu") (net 34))
 (segment (start 196.52 49.2) (end 193.98 49.2) (width 0.25) (layer "F.Cu") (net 34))
 (segment (start 191.6294 50.3753) (end 192.8047 49.2) (width 0.25) (layer "F.Cu") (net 34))
 (segment (start 138.1 97.46) (end 139.2753 97.46) (width 0.25) (layer "F.Cu") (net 34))
 (segment (start 139.2753 97.46) (end 139.2753 97.0927) (width 0.25) (layer "F.Cu") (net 34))
 (segment (start 129.6547 98.6353) (end 133.5768 98.6353) (width 0.25) (layer "F.Cu") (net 38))
 (segment (start 122.575 105.715) (end 129.6547 98.6353) (width 0.25) (layer "F.Cu") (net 38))
 (segment (start 134.3847 97.8274) (end 134.3847 97.46) (width 0.25) (layer "F.Cu") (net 38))
 (segment (start 133.5768 98.6353) (end 134.3847 97.8274) (width 0.25) (layer "F.Cu") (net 38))
 (segment (start 135.56 97.46) (end 134.3847 97.46) (width 0.25) (layer "F.Cu") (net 38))
 (segment (start 121.305 106.985) (end 121.2437 106.985) (width 0.25) (layer "B.Cu") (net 38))
 (segment (start 121.2437 106.985) (end 120.035 105.7763) (width 0.25) (layer "B.Cu") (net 38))
 (segment (start 122.575 105.715) (end 121.305 106.985) (width 0.25) (layer "B.Cu") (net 38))
 (segment (start 120.325 132.385) (end 121.2437 131.4663) (width 0.25) (layer "B.Cu") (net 38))
 (segment (start 121.2437 131.4663) (end 121.2437 106.985) (width 0.25) (layer "B.Cu") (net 38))
 (segment (start 120.035 105.7763) (end 120.035 105.715) (width 0.25) (layer "B.Cu") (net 38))
 (segment (start 181.8368 50.3753) (end 182.6447 49.5674) (width 0.25) (layer "F.Cu") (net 57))
 (segment (start 122.5113 49.5673) (end 123.3193 50.3753) (width 0.25) (layer "F.Cu") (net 57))
 (segment (start 183.82 49.2) (end 182.6447 49.2) (width 0.25) (layer "F.Cu") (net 57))
 (segment (start 121.336 49.2) (end 122.5113 49.2) (width 0.25) (layer "F.Cu") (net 57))
 (segment (start 123.3193 50.3753) (end 181.8368 50.3753) (width 0.25) (layer "F.Cu") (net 57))
 (segment (start 122.5113 49.2) (end 122.5113 49.5673) (width 0.25) (layer "F.Cu") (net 57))
 (segment (start 182.6447 49.5674) (end 182.6447 49.2) (width 0.25) (layer "F.Cu") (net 57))
 (segment (start 185.1847 48.8327) (end 184.3767 48.0247) (width 0.25) (layer "F.Cu") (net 56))
 (segment (start 118.796 49.2) (end 119.9713 49.2) (width 0.25) (layer "F.Cu") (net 56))
 (segment (start 186.36 49.2) (end 185.1847 49.2) (width 0.25) (layer "F.Cu") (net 56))
 (segment (start 184.3767 48.0247) (end 120.7792 48.0247) (width 0.25) (layer "F.Cu") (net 56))
 (segment (start 185.1847 49.2) (end 185.1847 48.8327) (width 0.25) (layer "F.Cu") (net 56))
 (segment (start 120.7792 48.0247) (end 119.9713 48.8326) (width 0.25) (layer "F.Cu") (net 56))
 (segment (start 119.9713 48.8326) (end 119.9713 49.2) (width 0.25) (layer "F.Cu") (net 56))
 (segment (start 130.195 126.035) (end 130.195 127.595) (width 0.25) (layer "B.Cu") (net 79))
 (segment (start 130.195 127.595) (end 125.405 132.385) (width 0.25) (layer "B.Cu") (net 79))
 (segment (start 128.925 124.765) (end 128.925 100.0401) (width 0.25) (layer "B.Cu") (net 62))
 (segment (start 136.576 49.2) (end 136.576 50.3753) (width 0.25) (layer "B.Cu") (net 62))
 (segment (start 129.1154 99.8497) (end 129.1154 57.8359) (width 0.25) (layer "B.Cu") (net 62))
 (segment (start 128.925 100.0401) (end 129.1154 99.8497) (width 0.25) (layer "B.Cu") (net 62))
 (segment (start 129.1154 57.8359) (end 136.576 50.3753) (width 0.25) (layer "B.Cu") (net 62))
 (segment (start 127.655 126.035) (end 128.925 124.765) (width 0.25) (layer "B.Cu") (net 62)))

